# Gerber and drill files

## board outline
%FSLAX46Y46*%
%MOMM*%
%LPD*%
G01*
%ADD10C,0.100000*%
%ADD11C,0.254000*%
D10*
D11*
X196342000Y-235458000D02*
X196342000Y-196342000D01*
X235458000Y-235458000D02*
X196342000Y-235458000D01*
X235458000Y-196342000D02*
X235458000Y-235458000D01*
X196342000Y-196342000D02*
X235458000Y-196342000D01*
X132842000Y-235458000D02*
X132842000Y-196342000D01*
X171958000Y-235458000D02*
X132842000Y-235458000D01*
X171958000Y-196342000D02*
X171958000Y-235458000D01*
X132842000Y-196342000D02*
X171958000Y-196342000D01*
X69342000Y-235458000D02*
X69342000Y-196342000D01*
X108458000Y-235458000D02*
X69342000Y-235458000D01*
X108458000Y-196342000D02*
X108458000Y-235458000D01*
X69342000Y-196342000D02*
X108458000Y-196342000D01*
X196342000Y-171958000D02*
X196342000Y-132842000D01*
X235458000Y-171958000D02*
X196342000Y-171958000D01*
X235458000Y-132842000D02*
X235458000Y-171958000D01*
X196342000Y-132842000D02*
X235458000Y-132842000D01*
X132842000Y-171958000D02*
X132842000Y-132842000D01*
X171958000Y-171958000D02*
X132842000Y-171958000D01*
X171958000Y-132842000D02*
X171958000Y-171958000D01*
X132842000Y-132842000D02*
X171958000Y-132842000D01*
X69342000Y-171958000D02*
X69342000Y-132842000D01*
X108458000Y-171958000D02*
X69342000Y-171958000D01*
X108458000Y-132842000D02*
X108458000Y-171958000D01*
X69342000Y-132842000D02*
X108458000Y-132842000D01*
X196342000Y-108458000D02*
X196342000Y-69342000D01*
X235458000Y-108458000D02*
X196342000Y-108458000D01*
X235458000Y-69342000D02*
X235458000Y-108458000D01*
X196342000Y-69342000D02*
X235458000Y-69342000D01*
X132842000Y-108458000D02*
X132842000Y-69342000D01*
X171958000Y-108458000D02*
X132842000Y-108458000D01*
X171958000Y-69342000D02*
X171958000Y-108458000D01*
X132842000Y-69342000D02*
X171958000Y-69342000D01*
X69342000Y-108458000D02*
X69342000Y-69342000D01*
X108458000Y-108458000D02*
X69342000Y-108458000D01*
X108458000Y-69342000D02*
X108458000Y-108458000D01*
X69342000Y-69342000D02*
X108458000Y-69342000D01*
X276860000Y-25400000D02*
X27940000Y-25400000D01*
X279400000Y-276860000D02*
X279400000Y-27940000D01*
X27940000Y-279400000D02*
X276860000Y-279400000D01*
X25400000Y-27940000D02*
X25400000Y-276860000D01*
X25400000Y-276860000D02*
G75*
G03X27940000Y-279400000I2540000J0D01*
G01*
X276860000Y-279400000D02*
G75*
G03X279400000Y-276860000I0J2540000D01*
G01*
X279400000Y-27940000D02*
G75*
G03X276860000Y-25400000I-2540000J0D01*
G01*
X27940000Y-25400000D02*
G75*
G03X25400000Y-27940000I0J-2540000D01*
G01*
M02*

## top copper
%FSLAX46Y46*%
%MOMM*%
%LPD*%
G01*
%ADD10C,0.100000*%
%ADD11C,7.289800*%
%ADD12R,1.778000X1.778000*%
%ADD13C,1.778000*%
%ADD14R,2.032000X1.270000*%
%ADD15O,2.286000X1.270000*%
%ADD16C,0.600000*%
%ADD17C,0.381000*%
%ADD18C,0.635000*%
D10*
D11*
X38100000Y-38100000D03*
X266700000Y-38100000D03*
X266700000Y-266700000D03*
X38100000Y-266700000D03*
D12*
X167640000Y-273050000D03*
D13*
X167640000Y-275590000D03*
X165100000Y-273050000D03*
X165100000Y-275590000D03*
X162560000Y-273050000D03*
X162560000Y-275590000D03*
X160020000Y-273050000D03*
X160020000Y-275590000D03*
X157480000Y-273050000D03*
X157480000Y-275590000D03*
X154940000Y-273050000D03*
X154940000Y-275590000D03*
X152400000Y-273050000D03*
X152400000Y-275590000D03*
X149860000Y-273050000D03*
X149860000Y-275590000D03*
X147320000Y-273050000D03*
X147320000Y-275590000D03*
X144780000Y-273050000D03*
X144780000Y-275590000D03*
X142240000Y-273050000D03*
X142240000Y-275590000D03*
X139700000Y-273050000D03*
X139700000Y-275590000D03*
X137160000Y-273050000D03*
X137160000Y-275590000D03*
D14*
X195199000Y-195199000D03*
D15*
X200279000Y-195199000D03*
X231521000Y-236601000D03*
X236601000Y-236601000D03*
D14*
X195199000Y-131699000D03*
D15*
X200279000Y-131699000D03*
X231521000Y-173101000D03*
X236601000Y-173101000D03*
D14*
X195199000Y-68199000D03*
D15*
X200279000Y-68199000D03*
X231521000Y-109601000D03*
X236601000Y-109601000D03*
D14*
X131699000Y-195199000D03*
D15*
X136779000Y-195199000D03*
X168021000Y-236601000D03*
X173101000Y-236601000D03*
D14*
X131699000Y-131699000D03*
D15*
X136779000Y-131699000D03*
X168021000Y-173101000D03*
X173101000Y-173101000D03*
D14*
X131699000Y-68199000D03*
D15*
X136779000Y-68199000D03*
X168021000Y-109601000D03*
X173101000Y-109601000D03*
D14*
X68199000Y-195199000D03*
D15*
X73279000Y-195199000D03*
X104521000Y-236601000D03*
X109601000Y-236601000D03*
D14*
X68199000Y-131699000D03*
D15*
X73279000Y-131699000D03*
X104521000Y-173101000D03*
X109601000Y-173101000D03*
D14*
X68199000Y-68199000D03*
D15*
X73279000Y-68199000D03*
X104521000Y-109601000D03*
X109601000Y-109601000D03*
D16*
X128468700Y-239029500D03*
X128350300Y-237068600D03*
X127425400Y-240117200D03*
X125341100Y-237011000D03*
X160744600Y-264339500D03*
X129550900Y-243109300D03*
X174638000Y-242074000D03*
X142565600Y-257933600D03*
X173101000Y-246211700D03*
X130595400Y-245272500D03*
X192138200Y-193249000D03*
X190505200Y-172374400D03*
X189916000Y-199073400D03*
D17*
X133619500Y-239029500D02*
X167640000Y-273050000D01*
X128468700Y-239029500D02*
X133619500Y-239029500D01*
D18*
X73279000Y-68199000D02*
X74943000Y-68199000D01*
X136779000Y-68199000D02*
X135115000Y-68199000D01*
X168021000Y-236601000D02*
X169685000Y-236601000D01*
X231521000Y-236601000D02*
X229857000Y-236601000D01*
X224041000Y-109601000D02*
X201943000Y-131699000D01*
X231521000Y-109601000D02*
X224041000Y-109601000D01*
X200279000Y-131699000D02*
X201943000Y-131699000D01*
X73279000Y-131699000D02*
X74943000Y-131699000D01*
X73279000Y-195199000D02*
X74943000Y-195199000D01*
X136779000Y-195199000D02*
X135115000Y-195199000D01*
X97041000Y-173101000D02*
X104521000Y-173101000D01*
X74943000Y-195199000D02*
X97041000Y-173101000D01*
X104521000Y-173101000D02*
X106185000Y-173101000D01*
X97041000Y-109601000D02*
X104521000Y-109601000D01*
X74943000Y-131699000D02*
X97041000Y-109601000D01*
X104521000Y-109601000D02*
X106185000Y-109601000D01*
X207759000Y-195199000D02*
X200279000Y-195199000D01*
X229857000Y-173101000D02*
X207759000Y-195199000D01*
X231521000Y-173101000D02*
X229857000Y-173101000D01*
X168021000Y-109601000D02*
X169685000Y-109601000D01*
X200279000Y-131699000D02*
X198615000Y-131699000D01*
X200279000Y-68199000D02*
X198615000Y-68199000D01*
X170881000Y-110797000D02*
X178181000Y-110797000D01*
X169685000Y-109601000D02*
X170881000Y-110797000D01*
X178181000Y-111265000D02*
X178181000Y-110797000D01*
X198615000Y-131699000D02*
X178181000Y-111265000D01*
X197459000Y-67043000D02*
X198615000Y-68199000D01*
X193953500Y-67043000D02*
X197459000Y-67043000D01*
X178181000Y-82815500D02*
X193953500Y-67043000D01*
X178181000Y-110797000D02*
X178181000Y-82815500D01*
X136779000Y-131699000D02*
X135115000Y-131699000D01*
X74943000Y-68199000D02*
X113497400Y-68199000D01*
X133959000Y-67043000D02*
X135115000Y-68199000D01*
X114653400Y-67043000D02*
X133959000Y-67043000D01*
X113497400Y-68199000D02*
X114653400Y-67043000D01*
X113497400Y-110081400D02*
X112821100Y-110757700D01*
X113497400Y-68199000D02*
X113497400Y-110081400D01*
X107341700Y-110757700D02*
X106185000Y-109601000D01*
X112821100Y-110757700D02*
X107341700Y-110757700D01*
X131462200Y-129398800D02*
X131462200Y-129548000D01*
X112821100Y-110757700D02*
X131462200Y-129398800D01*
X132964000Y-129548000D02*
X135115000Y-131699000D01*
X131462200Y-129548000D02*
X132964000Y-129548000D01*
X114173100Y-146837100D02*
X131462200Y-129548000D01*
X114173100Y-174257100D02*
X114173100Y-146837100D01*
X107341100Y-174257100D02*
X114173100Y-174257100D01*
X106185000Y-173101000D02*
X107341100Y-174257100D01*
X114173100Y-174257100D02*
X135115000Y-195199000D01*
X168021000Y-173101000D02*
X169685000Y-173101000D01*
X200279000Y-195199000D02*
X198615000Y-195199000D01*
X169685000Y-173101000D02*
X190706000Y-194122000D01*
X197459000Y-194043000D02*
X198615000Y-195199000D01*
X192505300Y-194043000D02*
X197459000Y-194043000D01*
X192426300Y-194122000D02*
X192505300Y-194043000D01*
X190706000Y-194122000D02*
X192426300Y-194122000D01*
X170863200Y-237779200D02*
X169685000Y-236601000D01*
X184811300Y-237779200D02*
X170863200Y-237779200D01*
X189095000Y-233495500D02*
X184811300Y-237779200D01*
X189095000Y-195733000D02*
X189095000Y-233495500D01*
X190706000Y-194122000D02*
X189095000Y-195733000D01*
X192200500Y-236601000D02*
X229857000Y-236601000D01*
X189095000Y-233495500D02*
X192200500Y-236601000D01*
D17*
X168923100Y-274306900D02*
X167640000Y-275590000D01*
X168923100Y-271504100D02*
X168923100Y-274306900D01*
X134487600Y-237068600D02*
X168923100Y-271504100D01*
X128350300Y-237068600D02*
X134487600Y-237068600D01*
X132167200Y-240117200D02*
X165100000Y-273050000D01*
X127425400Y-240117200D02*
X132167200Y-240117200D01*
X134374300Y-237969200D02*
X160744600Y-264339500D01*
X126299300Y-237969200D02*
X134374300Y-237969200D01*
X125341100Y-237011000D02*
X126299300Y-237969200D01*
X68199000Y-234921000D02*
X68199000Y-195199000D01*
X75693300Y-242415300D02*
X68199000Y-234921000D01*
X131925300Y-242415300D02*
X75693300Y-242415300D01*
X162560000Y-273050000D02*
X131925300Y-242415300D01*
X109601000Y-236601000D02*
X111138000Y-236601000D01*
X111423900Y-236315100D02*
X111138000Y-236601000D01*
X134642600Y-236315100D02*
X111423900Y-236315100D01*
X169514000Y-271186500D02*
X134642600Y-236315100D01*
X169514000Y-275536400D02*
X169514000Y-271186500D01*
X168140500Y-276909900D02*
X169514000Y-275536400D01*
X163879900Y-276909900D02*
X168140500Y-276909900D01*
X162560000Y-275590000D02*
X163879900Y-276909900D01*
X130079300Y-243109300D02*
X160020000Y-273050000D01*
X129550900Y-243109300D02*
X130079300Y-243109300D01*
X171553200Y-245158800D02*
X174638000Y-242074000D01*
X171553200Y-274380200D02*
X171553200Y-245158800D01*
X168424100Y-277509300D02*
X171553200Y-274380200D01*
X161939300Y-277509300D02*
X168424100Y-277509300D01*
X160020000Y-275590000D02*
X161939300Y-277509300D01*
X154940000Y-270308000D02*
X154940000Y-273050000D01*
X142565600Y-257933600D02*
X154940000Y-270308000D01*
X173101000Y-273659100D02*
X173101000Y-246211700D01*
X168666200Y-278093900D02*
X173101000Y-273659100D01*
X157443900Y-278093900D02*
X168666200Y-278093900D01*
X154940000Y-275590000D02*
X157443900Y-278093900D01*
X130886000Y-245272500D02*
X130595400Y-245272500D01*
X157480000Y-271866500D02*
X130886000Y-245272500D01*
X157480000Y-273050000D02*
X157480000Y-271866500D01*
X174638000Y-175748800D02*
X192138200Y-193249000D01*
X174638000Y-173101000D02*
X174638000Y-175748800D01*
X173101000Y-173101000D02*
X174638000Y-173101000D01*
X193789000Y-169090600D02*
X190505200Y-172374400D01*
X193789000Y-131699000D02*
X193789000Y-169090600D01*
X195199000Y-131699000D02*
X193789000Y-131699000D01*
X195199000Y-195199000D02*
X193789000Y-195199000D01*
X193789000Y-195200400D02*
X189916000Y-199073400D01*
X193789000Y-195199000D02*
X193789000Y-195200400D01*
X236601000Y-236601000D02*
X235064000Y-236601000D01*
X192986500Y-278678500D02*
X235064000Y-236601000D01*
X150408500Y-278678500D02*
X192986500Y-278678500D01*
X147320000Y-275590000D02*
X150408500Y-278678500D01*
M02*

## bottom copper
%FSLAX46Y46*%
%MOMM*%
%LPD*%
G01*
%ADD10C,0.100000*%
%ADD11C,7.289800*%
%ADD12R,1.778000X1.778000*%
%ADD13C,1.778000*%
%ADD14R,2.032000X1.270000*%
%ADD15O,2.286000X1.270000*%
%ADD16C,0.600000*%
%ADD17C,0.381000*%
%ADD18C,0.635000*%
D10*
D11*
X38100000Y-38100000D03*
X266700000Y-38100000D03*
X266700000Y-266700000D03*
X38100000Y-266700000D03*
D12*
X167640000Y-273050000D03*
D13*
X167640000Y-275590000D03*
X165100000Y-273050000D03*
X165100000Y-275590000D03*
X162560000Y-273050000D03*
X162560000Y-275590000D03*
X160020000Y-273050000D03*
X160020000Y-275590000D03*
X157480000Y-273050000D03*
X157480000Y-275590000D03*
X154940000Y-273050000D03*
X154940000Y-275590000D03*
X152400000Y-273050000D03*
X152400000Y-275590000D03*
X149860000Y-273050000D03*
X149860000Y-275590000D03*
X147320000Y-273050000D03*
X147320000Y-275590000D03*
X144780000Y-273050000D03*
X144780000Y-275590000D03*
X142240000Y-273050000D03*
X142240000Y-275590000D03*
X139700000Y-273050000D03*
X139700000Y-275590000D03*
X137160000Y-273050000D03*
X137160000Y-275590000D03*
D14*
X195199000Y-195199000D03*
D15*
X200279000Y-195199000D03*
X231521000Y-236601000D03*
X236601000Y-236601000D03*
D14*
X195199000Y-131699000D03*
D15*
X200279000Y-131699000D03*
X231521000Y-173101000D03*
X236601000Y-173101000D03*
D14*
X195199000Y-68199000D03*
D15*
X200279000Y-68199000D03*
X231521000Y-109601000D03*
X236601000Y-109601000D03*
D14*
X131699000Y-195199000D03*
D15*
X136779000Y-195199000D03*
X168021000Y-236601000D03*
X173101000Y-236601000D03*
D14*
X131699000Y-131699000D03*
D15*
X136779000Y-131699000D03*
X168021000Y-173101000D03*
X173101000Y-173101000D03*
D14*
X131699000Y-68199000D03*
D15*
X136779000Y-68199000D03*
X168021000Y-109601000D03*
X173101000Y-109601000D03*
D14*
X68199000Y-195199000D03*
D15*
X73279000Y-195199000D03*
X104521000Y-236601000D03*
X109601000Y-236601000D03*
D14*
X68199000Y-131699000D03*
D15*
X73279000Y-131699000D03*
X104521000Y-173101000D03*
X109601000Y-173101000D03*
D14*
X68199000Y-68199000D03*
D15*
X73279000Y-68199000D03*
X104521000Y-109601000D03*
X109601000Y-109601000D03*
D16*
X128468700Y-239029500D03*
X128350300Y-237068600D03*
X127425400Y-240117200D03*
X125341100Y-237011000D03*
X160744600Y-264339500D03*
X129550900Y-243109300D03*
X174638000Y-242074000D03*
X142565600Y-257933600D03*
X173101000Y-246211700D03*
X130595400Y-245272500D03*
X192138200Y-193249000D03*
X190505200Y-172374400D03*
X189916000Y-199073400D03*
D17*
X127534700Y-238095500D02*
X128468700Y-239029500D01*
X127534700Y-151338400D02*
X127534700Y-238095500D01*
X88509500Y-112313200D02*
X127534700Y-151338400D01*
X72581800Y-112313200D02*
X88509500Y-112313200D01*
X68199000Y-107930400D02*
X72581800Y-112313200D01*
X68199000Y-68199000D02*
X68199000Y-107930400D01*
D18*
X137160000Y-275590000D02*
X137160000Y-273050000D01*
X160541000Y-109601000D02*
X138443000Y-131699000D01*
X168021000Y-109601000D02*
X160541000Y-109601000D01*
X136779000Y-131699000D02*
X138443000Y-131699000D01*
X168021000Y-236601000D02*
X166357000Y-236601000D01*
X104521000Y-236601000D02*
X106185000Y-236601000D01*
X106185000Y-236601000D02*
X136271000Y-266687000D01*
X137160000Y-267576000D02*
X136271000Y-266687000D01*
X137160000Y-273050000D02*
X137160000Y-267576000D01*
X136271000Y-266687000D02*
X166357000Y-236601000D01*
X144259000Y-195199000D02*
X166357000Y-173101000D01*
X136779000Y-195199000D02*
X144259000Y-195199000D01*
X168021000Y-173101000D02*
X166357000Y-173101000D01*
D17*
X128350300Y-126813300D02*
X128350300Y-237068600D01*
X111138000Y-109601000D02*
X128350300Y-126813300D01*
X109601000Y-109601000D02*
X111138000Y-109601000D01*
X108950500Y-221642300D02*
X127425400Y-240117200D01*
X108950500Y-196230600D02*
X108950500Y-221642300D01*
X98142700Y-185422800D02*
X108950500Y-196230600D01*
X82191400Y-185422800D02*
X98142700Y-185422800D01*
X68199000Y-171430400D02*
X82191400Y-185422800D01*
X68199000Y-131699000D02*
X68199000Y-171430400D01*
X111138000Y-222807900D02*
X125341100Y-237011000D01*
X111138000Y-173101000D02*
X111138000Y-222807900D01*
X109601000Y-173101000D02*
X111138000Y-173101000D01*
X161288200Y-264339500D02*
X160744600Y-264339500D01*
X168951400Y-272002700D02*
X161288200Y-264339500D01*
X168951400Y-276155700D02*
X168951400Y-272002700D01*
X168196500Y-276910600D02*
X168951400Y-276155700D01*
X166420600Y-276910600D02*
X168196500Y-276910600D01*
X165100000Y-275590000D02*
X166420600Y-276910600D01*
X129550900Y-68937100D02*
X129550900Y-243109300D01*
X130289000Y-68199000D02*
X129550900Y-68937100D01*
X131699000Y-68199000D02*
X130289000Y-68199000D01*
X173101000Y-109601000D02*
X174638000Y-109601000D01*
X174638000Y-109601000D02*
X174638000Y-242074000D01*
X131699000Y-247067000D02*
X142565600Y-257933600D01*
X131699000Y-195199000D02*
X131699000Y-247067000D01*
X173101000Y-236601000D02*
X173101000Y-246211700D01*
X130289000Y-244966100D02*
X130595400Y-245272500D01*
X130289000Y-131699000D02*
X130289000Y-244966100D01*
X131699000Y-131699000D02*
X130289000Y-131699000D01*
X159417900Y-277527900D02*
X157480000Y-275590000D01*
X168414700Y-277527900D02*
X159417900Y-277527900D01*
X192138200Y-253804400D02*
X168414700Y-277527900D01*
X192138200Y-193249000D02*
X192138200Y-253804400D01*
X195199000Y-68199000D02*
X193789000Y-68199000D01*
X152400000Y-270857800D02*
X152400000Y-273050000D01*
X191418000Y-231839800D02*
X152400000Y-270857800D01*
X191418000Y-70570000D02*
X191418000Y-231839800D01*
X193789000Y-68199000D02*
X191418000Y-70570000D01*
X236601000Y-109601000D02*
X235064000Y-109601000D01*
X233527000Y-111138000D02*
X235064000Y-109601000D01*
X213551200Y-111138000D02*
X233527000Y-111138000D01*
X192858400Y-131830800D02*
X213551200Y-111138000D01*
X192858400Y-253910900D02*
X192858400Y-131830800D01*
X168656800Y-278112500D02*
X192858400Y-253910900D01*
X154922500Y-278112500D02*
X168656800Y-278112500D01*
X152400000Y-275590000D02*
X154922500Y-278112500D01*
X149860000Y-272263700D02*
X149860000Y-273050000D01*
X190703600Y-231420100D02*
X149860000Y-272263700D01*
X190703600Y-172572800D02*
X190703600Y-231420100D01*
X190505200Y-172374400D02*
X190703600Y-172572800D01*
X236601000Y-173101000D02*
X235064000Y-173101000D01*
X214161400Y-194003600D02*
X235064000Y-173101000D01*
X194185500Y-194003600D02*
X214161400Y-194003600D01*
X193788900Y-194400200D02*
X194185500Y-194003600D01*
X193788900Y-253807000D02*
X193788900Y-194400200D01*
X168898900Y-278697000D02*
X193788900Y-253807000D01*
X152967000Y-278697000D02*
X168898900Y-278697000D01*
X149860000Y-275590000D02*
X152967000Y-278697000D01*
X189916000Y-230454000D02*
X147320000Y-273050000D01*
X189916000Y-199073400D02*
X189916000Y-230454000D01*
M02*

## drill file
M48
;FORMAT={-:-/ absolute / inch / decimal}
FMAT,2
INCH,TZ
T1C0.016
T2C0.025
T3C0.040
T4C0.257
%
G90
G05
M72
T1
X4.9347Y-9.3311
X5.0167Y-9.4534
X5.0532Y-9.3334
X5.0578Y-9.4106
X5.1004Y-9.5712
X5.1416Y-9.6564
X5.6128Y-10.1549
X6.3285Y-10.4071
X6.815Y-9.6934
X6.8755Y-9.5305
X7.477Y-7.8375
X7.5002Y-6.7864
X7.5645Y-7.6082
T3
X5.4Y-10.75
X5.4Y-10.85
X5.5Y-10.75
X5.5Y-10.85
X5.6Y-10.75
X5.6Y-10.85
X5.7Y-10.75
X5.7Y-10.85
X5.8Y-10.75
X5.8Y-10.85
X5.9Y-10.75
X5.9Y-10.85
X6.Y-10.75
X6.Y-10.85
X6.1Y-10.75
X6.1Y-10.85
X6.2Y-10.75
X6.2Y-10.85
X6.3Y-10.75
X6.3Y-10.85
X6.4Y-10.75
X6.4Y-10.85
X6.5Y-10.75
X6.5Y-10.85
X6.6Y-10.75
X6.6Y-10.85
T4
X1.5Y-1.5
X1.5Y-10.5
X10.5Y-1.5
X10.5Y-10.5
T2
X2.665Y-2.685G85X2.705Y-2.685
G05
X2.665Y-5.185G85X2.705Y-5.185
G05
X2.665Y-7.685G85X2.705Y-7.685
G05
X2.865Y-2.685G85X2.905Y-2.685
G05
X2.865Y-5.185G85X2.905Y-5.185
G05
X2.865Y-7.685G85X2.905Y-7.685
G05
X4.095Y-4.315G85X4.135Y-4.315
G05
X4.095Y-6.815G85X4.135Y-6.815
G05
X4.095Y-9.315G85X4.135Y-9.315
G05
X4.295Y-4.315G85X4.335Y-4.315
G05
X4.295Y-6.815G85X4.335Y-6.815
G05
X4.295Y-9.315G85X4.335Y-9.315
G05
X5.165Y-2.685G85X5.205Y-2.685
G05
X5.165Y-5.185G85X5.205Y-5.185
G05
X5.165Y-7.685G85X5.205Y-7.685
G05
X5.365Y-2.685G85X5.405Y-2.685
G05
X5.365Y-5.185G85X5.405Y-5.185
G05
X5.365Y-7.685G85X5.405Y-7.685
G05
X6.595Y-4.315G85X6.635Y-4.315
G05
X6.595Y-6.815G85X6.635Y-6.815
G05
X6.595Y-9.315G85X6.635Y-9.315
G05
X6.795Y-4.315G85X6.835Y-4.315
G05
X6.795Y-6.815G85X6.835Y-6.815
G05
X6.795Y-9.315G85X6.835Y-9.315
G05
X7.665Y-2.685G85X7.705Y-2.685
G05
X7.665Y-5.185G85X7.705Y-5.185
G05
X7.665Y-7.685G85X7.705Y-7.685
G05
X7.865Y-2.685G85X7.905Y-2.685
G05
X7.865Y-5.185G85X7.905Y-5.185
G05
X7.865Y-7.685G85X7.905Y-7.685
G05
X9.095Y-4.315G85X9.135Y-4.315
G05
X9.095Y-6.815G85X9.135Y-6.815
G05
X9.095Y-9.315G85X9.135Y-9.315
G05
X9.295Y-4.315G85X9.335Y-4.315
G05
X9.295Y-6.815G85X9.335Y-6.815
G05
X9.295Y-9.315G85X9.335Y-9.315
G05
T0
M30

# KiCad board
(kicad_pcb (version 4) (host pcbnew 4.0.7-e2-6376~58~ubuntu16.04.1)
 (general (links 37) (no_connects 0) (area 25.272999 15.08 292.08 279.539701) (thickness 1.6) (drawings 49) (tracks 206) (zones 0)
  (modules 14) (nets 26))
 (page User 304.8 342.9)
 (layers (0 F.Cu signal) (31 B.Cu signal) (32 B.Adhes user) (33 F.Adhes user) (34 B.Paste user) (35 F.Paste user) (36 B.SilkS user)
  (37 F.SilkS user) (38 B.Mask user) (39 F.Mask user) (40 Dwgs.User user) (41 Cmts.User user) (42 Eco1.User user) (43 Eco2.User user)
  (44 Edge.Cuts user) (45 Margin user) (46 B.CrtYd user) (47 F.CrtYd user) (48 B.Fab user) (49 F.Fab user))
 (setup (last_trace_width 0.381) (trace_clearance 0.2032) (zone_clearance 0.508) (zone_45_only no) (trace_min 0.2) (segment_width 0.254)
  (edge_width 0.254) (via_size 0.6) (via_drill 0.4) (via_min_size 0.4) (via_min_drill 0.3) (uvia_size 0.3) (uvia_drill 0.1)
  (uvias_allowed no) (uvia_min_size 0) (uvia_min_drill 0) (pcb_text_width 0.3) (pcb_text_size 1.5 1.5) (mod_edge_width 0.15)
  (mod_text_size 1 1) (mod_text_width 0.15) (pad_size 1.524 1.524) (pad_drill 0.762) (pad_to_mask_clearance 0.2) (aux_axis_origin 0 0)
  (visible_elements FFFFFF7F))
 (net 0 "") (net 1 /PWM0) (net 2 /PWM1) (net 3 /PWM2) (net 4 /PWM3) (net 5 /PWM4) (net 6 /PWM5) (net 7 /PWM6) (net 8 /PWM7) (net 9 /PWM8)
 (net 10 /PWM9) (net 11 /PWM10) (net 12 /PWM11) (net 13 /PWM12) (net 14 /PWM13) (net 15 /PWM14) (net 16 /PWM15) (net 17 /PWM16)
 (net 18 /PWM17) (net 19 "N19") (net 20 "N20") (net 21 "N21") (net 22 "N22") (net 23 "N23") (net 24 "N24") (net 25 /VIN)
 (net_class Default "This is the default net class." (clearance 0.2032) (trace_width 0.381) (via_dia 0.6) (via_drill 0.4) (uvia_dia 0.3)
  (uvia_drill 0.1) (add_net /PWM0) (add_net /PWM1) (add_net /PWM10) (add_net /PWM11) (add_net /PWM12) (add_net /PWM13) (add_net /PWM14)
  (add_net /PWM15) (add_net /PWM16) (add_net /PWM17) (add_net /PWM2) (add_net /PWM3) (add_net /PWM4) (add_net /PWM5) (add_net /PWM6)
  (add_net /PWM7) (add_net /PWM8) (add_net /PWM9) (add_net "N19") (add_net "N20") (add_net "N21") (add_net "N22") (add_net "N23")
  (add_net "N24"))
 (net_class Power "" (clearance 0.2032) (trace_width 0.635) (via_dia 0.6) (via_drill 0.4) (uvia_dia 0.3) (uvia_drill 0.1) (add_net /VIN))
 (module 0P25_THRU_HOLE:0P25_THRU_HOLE (layer F.Cu) (at 38.1 38.1)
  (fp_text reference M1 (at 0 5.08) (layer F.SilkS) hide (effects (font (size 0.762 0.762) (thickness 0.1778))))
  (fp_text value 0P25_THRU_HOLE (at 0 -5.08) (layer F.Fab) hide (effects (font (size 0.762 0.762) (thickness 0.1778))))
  (pad "" thru_hole circle (at 0 0) (size 7.2898 7.2898) (drill 6.5278) (layers *.Cu *.Mask)))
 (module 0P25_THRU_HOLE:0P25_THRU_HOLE (layer F.Cu) (at 266.7 38.1)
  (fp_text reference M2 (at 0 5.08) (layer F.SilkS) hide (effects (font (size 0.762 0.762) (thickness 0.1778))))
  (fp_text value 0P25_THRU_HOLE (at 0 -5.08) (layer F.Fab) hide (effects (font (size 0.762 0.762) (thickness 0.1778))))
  (pad "" thru_hole circle (at 0 0) (size 7.2898 7.2898) (drill 6.5278) (layers *.Cu *.Mask)))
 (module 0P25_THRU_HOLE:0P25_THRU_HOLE (layer F.Cu) (at 266.7 266.7)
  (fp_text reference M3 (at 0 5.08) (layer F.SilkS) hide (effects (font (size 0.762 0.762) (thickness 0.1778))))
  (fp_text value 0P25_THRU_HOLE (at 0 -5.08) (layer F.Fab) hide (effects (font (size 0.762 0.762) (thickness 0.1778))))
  (pad "" thru_hole circle (at 0 0) (size 7.2898 7.2898) (drill 6.5278) (layers *.Cu *.Mask)))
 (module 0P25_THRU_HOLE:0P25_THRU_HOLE (layer F.Cu) (at 38.1 266.7)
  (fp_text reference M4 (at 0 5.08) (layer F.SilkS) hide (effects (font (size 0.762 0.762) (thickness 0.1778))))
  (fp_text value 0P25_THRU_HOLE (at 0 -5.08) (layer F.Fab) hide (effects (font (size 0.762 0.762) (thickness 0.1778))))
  (pad "" thru_hole circle (at 0 0) (size 7.2898 7.2898) (drill 6.5278) (layers *.Cu *.Mask)))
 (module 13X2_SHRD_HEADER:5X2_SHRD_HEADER (layer F.Cu) (at 152.4 274.32 180)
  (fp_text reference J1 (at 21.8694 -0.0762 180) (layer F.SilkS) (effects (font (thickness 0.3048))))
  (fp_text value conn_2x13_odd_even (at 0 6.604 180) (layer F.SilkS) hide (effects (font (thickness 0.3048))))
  (pad 1 thru_hole rect (at -15.24 1.27 180) (size 1.778 1.778) (drill 1.016) (layers *.Cu *.Mask F.SilkS) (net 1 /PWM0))
  (pad 2 thru_hole circle (at -15.24 -1.27 180) (size 1.778 1.778) (drill 1.016) (layers *.Cu *.Mask F.SilkS) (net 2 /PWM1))
  (pad 3 thru_hole circle (at -12.7 1.27 180) (size 1.778 1.778) (drill 1.016) (layers *.Cu *.Mask F.SilkS) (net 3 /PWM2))
  (pad 4 thru_hole circle (at -12.7 -1.27 180) (size 1.778 1.778) (drill 1.016) (layers *.Cu *.Mask F.SilkS) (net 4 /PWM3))
  (pad 5 thru_hole circle (at -10.16 1.27 180) (size 1.778 1.778) (drill 1.016) (layers *.Cu *.Mask F.SilkS) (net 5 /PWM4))
  (pad 6 thru_hole circle (at -10.16 -1.27 180) (size 1.778 1.778) (drill 1.016) (layers *.Cu *.Mask F.SilkS) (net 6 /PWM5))
  (pad 7 thru_hole circle (at -7.62 1.27 180) (size 1.778 1.778) (drill 1.016) (layers *.Cu *.Mask F.SilkS) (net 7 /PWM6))
  (pad 8 thru_hole circle (at -7.62 -1.27 180) (size 1.778 1.778) (drill 1.016) (layers *.Cu *.Mask F.SilkS) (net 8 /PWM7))
  (pad 9 thru_hole circle (at -5.08 1.27 180) (size 1.778 1.778) (drill 1.016) (layers *.Cu *.Mask F.SilkS) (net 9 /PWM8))
  (pad 10 thru_hole circle (at -5.08 -1.27 180) (size 1.778 1.778) (drill 1.016) (layers *.Cu *.Mask F.SilkS) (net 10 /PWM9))
  (pad 11 thru_hole circle (at -2.54 1.27 180) (size 1.778 1.778) (drill 1.016) (layers *.Cu *.Mask) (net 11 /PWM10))
  (pad 12 thru_hole circle (at -2.54 -1.27 180) (size 1.778 1.778) (drill 1.016) (layers *.Cu *.Mask) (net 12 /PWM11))
  (pad 13 thru_hole circle (at 0 1.27 180) (size 1.778 1.778) (drill 1.016) (layers *.Cu *.Mask) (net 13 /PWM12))
  (pad 14 thru_hole circle (at 0 -1.27 180) (size 1.778 1.778) (drill 1.016) (layers *.Cu *.Mask) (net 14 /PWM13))
  (pad 15 thru_hole circle (at 2.54 1.27 180) (size 1.778 1.778) (drill 1.016) (layers *.Cu *.Mask) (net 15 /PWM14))
  (pad 16 thru_hole circle (at 2.54 -1.27 180) (size 1.778 1.778) (drill 1.016) (layers *.Cu *.Mask) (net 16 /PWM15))
  (pad 17 thru_hole circle (at 5.08 1.27 180) (size 1.778 1.778) (drill 1.016) (layers *.Cu *.Mask) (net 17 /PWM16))
  (pad 18 thru_hole circle (at 5.08 -1.27 180) (size 1.778 1.778) (drill 1.016) (layers *.Cu *.Mask) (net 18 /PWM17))
  (pad 19 thru_hole circle (at 7.62 1.27 180) (size 1.778 1.778) (drill 1.016) (layers *.Cu *.Mask) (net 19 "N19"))
  (pad 20 thru_hole circle (at 7.62 -1.27 180) (size 1.778 1.778) (drill 1.016) (layers *.Cu *.Mask) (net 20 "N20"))
  (pad 21 thru_hole circle (at 10.16 1.27 180) (size 1.778 1.778) (drill 1.016) (layers *.Cu *.Mask) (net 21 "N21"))
  (pad 22 thru_hole circle (at 10.16 -1.27 180) (size 1.778 1.778) (drill 1.016) (layers *.Cu *.Mask) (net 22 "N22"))
  (pad 23 thru_hole circle (at 12.7 1.27 180) (size 1.778 1.778) (drill 1.016) (layers *.Cu *.Mask) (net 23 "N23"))
  (pad 24 thru_hole circle (at 12.7 -1.27 180) (size 1.778 1.778) (drill 1.016) (layers *.Cu *.Mask) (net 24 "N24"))
  (pad 25 thru_hole circle (at 15.24 1.27 180) (size 1.778 1.778) (drill 1.016) (layers *.Cu *.Mask) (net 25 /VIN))
  (pad 26 thru_hole circle (at 15.24 -1.27 180) (size 1.778 1.778) (drill 1.016) (layers *.Cu *.Mask) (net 25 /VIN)))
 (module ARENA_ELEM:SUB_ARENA (layer F.Cu) (at 215.9 215.9)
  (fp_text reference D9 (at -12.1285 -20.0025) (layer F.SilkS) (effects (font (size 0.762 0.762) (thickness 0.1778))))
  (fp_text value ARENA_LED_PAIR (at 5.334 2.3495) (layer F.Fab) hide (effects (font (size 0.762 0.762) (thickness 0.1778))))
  (pad 1 thru_hole rect (at -20.701 -20.701) (size 2.032 1.27) (drill oval 1.651 0.635) (layers *.Cu *.Mask) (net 17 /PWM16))
  (pad 2 thru_hole oval (at -15.621 -20.701) (size 2.286 1.27) (drill oval 1.651 0.635) (layers *.Cu *.Mask) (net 25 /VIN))
  (pad 4 thru_hole oval (at 15.621 20.701) (size 2.286 1.27) (drill oval 1.651 0.635) (layers *.Cu *.Mask) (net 25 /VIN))
  (pad 3 thru_hole oval (at 20.701 20.701) (size 2.286 1.27) (drill oval 1.651 0.635) (layers *.Cu *.Mask) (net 18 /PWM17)))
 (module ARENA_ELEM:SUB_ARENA (layer F.Cu) (at 215.9 152.4)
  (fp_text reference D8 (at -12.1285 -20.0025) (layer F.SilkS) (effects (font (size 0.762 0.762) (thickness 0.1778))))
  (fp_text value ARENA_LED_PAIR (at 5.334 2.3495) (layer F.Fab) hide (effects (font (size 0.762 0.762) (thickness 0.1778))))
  (pad 1 thru_hole rect (at -20.701 -20.701) (size 2.032 1.27) (drill oval 1.651 0.635) (layers *.Cu *.Mask) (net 15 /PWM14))
  (pad 2 thru_hole oval (at -15.621 -20.701) (size 2.286 1.27) (drill oval 1.651 0.635) (layers *.Cu *.Mask) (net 25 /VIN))
  (pad 4 thru_hole oval (at 15.621 20.701) (size 2.286 1.27) (drill oval 1.651 0.635) (layers *.Cu *.Mask) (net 25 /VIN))
  (pad 3 thru_hole oval (at 20.701 20.701) (size 2.286 1.27) (drill oval 1.651 0.635) (layers *.Cu *.Mask) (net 16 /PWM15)))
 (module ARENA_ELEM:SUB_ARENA (layer F.Cu) (at 215.9 88.9)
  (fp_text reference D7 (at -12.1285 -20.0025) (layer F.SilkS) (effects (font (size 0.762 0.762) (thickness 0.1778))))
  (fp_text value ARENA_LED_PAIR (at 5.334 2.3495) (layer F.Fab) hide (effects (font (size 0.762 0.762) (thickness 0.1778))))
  (pad 1 thru_hole rect (at -20.701 -20.701) (size 2.032 1.27) (drill oval 1.651 0.635) (layers *.Cu *.Mask) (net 13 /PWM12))
  (pad 2 thru_hole oval (at -15.621 -20.701) (size 2.286 1.27) (drill oval 1.651 0.635) (layers *.Cu *.Mask) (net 25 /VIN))
  (pad 4 thru_hole oval (at 15.621 20.701) (size 2.286 1.27) (drill oval 1.651 0.635) (layers *.Cu *.Mask) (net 25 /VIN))
  (pad 3 thru_hole oval (at 20.701 20.701) (size 2.286 1.27) (drill oval 1.651 0.635) (layers *.Cu *.Mask) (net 14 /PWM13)))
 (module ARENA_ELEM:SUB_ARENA (layer F.Cu) (at 152.4 215.9)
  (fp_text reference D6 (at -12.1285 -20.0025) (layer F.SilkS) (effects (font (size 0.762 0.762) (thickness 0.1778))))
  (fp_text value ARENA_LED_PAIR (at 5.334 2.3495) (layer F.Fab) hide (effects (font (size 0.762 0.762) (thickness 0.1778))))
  (pad 1 thru_hole rect (at -20.701 -20.701) (size 2.032 1.27) (drill oval 1.651 0.635) (layers *.Cu *.Mask) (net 11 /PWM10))
  (pad 2 thru_hole oval (at -15.621 -20.701) (size 2.286 1.27) (drill oval 1.651 0.635) (layers *.Cu *.Mask) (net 25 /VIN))
  (pad 4 thru_hole oval (at 15.621 20.701) (size 2.286 1.27) (drill oval 1.651 0.635) (layers *.Cu *.Mask) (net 25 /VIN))
  (pad 3 thru_hole oval (at 20.701 20.701) (size 2.286 1.27) (drill oval 1.651 0.635) (layers *.Cu *.Mask) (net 12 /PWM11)))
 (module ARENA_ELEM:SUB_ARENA (layer F.Cu) (at 152.4 152.4)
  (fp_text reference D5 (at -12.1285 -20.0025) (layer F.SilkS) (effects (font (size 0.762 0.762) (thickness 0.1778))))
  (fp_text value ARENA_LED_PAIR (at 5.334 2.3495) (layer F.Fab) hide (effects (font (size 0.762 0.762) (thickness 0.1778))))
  (pad 1 thru_hole rect (at -20.701 -20.701) (size 2.032 1.27) (drill oval 1.651 0.635) (layers *.Cu *.Mask) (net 9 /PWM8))
  (pad 2 thru_hole oval (at -15.621 -20.701) (size 2.286 1.27) (drill oval 1.651 0.635) (layers *.Cu *.Mask) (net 25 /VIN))
  (pad 4 thru_hole oval (at 15.621 20.701) (size 2.286 1.27) (drill oval 1.651 0.635) (layers *.Cu *.Mask) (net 25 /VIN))
  (pad 3 thru_hole oval (at 20.701 20.701) (size 2.286 1.27) (drill oval 1.651 0.635) (layers *.Cu *.Mask) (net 10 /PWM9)))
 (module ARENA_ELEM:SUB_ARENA (layer F.Cu) (at 152.4 88.9)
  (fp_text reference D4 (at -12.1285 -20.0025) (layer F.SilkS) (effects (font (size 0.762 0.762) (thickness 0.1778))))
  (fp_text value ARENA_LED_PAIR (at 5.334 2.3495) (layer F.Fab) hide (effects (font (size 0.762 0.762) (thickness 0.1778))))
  (pad 1 thru_hole rect (at -20.701 -20.701) (size 2.032 1.27) (drill oval 1.651 0.635) (layers *.Cu *.Mask) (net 7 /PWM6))
  (pad 2 thru_hole oval (at -15.621 -20.701) (size 2.286 1.27) (drill oval 1.651 0.635) (layers *.Cu *.Mask) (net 25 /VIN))
  (pad 4 thru_hole oval (at 15.621 20.701) (size 2.286 1.27) (drill oval 1.651 0.635) (layers *.Cu *.Mask) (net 25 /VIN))
  (pad 3 thru_hole oval (at 20.701 20.701) (size 2.286 1.27) (drill oval 1.651 0.635) (layers *.Cu *.Mask) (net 8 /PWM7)))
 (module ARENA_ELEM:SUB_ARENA (layer F.Cu) (at 88.9 215.9)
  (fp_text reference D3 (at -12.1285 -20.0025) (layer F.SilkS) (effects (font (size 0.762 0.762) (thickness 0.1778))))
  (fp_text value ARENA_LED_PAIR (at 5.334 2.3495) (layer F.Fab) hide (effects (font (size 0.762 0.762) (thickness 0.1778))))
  (pad 1 thru_hole rect (at -20.701 -20.701) (size 2.032 1.27) (drill oval 1.651 0.635) (layers *.Cu *.Mask) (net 5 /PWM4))
  (pad 2 thru_hole oval (at -15.621 -20.701) (size 2.286 1.27) (drill oval 1.651 0.635) (layers *.Cu *.Mask) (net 25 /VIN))
  (pad 4 thru_hole oval (at 15.621 20.701) (size 2.286 1.27) (drill oval 1.651 0.635) (layers *.Cu *.Mask) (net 25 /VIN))
  (pad 3 thru_hole oval (at 20.701 20.701) (size 2.286 1.27) (drill oval 1.651 0.635) (layers *.Cu *.Mask) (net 6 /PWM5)))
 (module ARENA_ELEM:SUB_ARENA (layer F.Cu) (at 88.9 152.4)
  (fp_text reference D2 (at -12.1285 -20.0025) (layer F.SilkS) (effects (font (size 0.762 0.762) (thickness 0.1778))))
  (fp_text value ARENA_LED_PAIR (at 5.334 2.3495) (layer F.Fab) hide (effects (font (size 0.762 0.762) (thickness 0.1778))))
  (pad 1 thru_hole rect (at -20.701 -20.701) (size 2.032 1.27) (drill oval 1.651 0.635) (layers *.Cu *.Mask) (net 3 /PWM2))
  (pad 2 thru_hole oval (at -15.621 -20.701) (size 2.286 1.27) (drill oval 1.651 0.635) (layers *.Cu *.Mask) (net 25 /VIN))
  (pad 4 thru_hole oval (at 15.621 20.701) (size 2.286 1.27) (drill oval 1.651 0.635) (layers *.Cu *.Mask) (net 25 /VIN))
  (pad 3 thru_hole oval (at 20.701 20.701) (size 2.286 1.27) (drill oval 1.651 0.635) (layers *.Cu *.Mask) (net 4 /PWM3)))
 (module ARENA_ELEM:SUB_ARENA (layer F.Cu) (at 88.9 88.9)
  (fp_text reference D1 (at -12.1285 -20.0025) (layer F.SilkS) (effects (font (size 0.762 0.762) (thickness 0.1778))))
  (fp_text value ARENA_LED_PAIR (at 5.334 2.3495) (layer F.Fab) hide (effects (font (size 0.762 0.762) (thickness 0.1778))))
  (pad 1 thru_hole rect (at -20.701 -20.701) (size 2.032 1.27) (drill oval 1.651 0.635) (layers *.Cu *.Mask) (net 1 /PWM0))
  (pad 2 thru_hole oval (at -15.621 -20.701) (size 2.286 1.27) (drill oval 1.651 0.635) (layers *.Cu *.Mask) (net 25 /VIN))
  (pad 4 thru_hole oval (at 15.621 20.701) (size 2.286 1.27) (drill oval 1.651 0.635) (layers *.Cu *.Mask) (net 25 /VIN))
  (pad 3 thru_hole oval (at 20.701 20.701) (size 2.286 1.27) (drill oval 1.651 0.635) (layers *.Cu *.Mask) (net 2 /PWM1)))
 (gr_line (start 196.342 235.458) (end 196.342 196.342) (angle 90) (layer Edge.Cuts) (width 0.254))
 (gr_line (start 235.458 235.458) (end 196.342 235.458) (angle 90) (layer Edge.Cuts) (width 0.254))
 (gr_line (start 235.458 196.342) (end 235.458 235.458) (angle 90) (layer Edge.Cuts) (width 0.254))
 (gr_line (start 196.342 196.342) (end 235.458 196.342) (angle 90) (layer Edge.Cuts) (width 0.254))
 (gr_line (start 132.842 235.458) (end 132.842 196.342) (angle 90) (layer Edge.Cuts) (width 0.254))
 (gr_line (start 171.958 235.458) (end 132.842 235.458) (angle 90) (layer Edge.Cuts) (width 0.254))
 (gr_line (start 171.958 196.342) (end 171.958 235.458) (angle 90) (layer Edge.Cuts) (width 0.254))
 (gr_line (start 132.842 196.342) (end 171.958 196.342) (angle 90) (layer Edge.Cuts) (width 0.254))
 (gr_line (start 69.342 235.458) (end 69.342 196.342) (angle 90) (layer Edge.Cuts) (width 0.254))
 (gr_line (start 108.458 235.458) (end 69.342 235.458) (angle 90) (layer Edge.Cuts) (width 0.254))
 (gr_line (start 108.458 196.342) (end 108.458 235.458) (angle 90) (layer Edge.Cuts) (width 0.254))
 (gr_line (start 69.342 196.342) (end 108.458 196.342) (angle 90) (layer Edge.Cuts) (width 0.254))
 (gr_line (start 196.342 171.958) (end 196.342 132.842) (angle 90) (layer Edge.Cuts) (width 0.254))
 (gr_line (start 235.458 171.958) (end 196.342 171.958) (angle 90) (layer Edge.Cuts) (width 0.254))
 (gr_line (start 235.458 132.842) (end 235.458 171.958) (angle 90) (layer Edge.Cuts) (width 0.254))
 (gr_line (start 196.342 132.842) (end 235.458 132.842) (angle 90) (layer Edge.Cuts) (width 0.254))
 (gr_line (start 132.842 171.958) (end 132.842 132.842) (angle 90) (layer Edge.Cuts) (width 0.254))
 (gr_line (start 171.958 171.958) (end 132.842 171.958) (angle 90) (layer Edge.Cuts) (width 0.254))
 (gr_line (start 171.958 132.842) (end 171.958 171.958) (angle 90) (layer Edge.Cuts) (width 0.254))
 (gr_line (start 132.842 132.842) (end 171.958 132.842) (angle 90) (layer Edge.Cuts) (width 0.254))
 (gr_line (start 69.342 171.958) (end 69.342 132.842) (angle 90) (layer Edge.Cuts) (width 0.254))
 (gr_line (start 108.458 171.958) (end 69.342 171.958) (angle 90) (layer Edge.Cuts) (width 0.254))
 (gr_line (start 108.458 132.842) (end 108.458 171.958) (angle 90) (layer Edge.Cuts) (width 0.254))
 (gr_line (start 69.342 132.842) (end 108.458 132.842) (angle 90) (layer Edge.Cuts) (width 0.254))
 (gr_line (start 196.342 108.458) (end 196.342 69.342) (angle 90) (layer Edge.Cuts) (width 0.254))
 (gr_line (start 235.458 108.458) (end 196.342 108.458) (angle 90) (layer Edge.Cuts) (width 0.254))
 (gr_line (start 235.458 69.342) (end 235.458 108.458) (angle 90) (layer Edge.Cuts) (width 0.254))
 (gr_line (start 196.342 69.342) (end 235.458 69.342) (angle 90) (layer Edge.Cuts) (width 0.254))
 (gr_line (start 132.842 108.458) (end 132.842 69.342) (angle 90) (layer Edge.Cuts) (width 0.254))
 (gr_line (start 171.958 108.458) (end 132.842 108.458) (angle 90) (layer Edge.Cuts) (width 0.254))
 (gr_line (start 171.958 69.342) (end 171.958 108.458) (angle 90) (layer Edge.Cuts) (width 0.254))
 (gr_line (start 132.842 69.342) (end 171.958 69.342) (angle 90) (layer Edge.Cuts) (width 0.254))
 (gr_line (start 69.342 108.458) (end 69.342 69.342) (angle 90) (layer Edge.Cuts) (width 0.254))
 (gr_line (start 108.458 108.458) (end 69.342 108.458) (angle 90) (layer Edge.Cuts) (width 0.254))
 (gr_line (start 108.458 69.342) (end 108.458 108.458) (angle 90) (layer Edge.Cuts) (width 0.254))
 (gr_line (start 69.342 69.342) (end 108.458 69.342) (angle 90) (layer Edge.Cuts) (width 0.254))
 (gr_line (start 276.86 25.4) (end 27.94 25.4) (angle 90) (layer Edge.Cuts) (width 0.254))
 (gr_line (start 279.4 276.86) (end 279.4 27.94) (angle 90) (layer Edge.Cuts) (width 0.254))
 (gr_line (start 27.94 279.4) (end 276.86 279.4) (angle 90) (layer Edge.Cuts) (width 0.254))
 (gr_line (start 25.4 27.94) (end 25.4 276.86) (angle 90) (layer Edge.Cuts) (width 0.254))
 (gr_arc (start 27.94 276.86) (end 27.94 279.4) (angle 90) (layer Edge.Cuts) (width 0.254))
 (gr_arc (start 276.86 276.86) (end 279.4 276.86) (angle 90) (layer Edge.Cuts) (width 0.254))
 (gr_arc (start 276.86 27.94) (end 276.86 25.4) (angle 90) (layer Edge.Cuts) (width 0.254))
 (gr_arc (start 27.94 27.94) (end 25.4 27.94) (angle 90) (layer Edge.Cuts) (width 0.254))
 (via (at 128.4687 239.0295) (size 0.6) (layers F.Cu B.Cu) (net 1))
 (segment (start 127.5347 238.0955) (end 128.4687 239.0295) (width 0.381) (layer B.Cu) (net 1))
 (segment (start 127.5347 151.3384) (end 127.5347 238.0955) (width 0.381) (layer B.Cu) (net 1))
 (segment (start 88.5095 112.3132) (end 127.5347 151.3384) (width 0.381) (layer B.Cu) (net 1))
 (segment (start 72.5818 112.3132) (end 88.5095 112.3132) (width 0.381) (layer B.Cu) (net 1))
 (segment (start 68.199 107.9304) (end 72.5818 112.3132) (width 0.381) (layer B.Cu) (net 1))
 (segment (start 68.199 68.199) (end 68.199 107.9304) (width 0.381) (layer B.Cu) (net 1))
 (segment (start 133.6195 239.0295) (end 167.64 273.05) (width 0.381) (layer F.Cu) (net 1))
 (segment (start 128.4687 239.0295) (end 133.6195 239.0295) (width 0.381) (layer F.Cu) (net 1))
 (segment (start 73.279 68.199) (end 74.943 68.199) (width 0.635) (layer F.Cu) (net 25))
 (segment (start 136.779 68.199) (end 135.115 68.199) (width 0.635) (layer F.Cu) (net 25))
 (segment (start 137.16 275.59) (end 137.16 273.05) (width 0.635) (layer B.Cu) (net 25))
 (segment (start 168.021 236.601) (end 169.685 236.601) (width 0.635) (layer F.Cu) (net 25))
 (segment (start 231.521 236.601) (end 229.857 236.601) (width 0.635) (layer F.Cu) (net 25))
 (segment (start 224.041 109.601) (end 201.943 131.699) (width 0.635) (layer F.Cu) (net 25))
 (segment (start 231.521 109.601) (end 224.041 109.601) (width 0.635) (layer F.Cu) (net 25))
 (segment (start 200.279 131.699) (end 201.943 131.699) (width 0.635) (layer F.Cu) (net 25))
 (segment (start 73.279 131.699) (end 74.943 131.699) (width 0.635) (layer F.Cu) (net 25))
 (segment (start 73.279 195.199) (end 74.943 195.199) (width 0.635) (layer F.Cu) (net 25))
 (segment (start 136.779 195.199) (end 135.115 195.199) (width 0.635) (layer F.Cu) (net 25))
 (segment (start 97.041 173.101) (end 104.521 173.101) (width 0.635) (layer F.Cu) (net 25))
 (segment (start 74.943 195.199) (end 97.041 173.101) (width 0.635) (layer F.Cu) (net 25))
 (segment (start 104.521 173.101) (end 106.185 173.101) (width 0.635) (layer F.Cu) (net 25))
 (segment (start 97.041 109.601) (end 104.521 109.601) (width 0.635) (layer F.Cu) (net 25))
 (segment (start 74.943 131.699) (end 97.041 109.601) (width 0.635) (layer F.Cu) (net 25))
 (segment (start 104.521 109.601) (end 106.185 109.601) (width 0.635) (layer F.Cu) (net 25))
 (segment (start 160.541 109.601) (end 138.443 131.699) (width 0.635) (layer B.Cu) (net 25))
 (segment (start 168.021 109.601) (end 160.541 109.601) (width 0.635) (layer B.Cu) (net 25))
 (segment (start 136.779 131.699) (end 138.443 131.699) (width 0.635) (layer B.Cu) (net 25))
 (segment (start 207.759 195.199) (end 200.279 195.199) (width 0.635) (layer F.Cu) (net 25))
 (segment (start 229.857 173.101) (end 207.759 195.199) (width 0.635) (layer F.Cu) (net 25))
 (segment (start 231.521 173.101) (end 229.857 173.101) (width 0.635) (layer F.Cu) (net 25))
 (segment (start 168.021 109.601) (end 169.685 109.601) (width 0.635) (layer F.Cu) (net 25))
 (segment (start 200.279 131.699) (end 198.615 131.699) (width 0.635) (layer F.Cu) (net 25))
 (segment (start 200.279 68.199) (end 198.615 68.199) (width 0.635) (layer F.Cu) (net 25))
 (segment (start 170.881 110.797) (end 178.181 110.797) (width 0.635) (layer F.Cu) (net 25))
 (segment (start 169.685 109.601) (end 170.881 110.797) (width 0.635) (layer F.Cu) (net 25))
 (segment (start 178.181 111.265) (end 178.181 110.797) (width 0.635) (layer F.Cu) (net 25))
 (segment (start 198.615 131.699) (end 178.181 111.265) (width 0.635) (layer F.Cu) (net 25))
 (segment (start 197.459 67.043) (end 198.615 68.199) (width 0.635) (layer F.Cu) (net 25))
 (segment (start 193.9535 67.043) (end 197.459 67.043) (width 0.635) (layer F.Cu) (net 25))
 (segment (start 178.181 82.8155) (end 193.9535 67.043) (width 0.635) (layer F.Cu) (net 25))
 (segment (start 178.181 110.797) (end 178.181 82.8155) (width 0.635) (layer F.Cu) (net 25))
 (segment (start 136.779 131.699) (end 135.115 131.699) (width 0.635) (layer F.Cu) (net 25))
 (segment (start 74.943 68.199) (end 113.4974 68.199) (width 0.635) (layer F.Cu) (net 25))
 (segment (start 133.959 67.043) (end 135.115 68.199) (width 0.635) (layer F.Cu) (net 25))
 (segment (start 114.6534 67.043) (end 133.959 67.043) (width 0.635) (layer F.Cu) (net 25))
 (segment (start 113.4974 68.199) (end 114.6534 67.043) (width 0.635) (layer F.Cu) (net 25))
 (segment (start 113.4974 110.0814) (end 112.8211 110.7577) (width 0.635) (layer F.Cu) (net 25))
 (segment (start 113.4974 68.199) (end 113.4974 110.0814) (width 0.635) (layer F.Cu) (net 25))
 (segment (start 107.3417 110.7577) (end 106.185 109.601) (width 0.635) (layer F.Cu) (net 25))
 (segment (start 112.8211 110.7577) (end 107.3417 110.7577) (width 0.635) (layer F.Cu) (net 25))
 (segment (start 131.4622 129.3988) (end 131.4622 129.548) (width 0.635) (layer F.Cu) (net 25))
 (segment (start 112.8211 110.7577) (end 131.4622 129.3988) (width 0.635) (layer F.Cu) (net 25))
 (segment (start 132.964 129.548) (end 135.115 131.699) (width 0.635) (layer F.Cu) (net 25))
 (segment (start 131.4622 129.548) (end 132.964 129.548) (width 0.635) (layer F.Cu) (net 25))
 (segment (start 114.1731 146.8371) (end 131.4622 129.548) (width 0.635) (layer F.Cu) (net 25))
 (segment (start 114.1731 174.2571) (end 114.1731 146.8371) (width 0.635) (layer F.Cu) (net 25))
 (segment (start 107.3411 174.2571) (end 114.1731 174.2571) (width 0.635) (layer F.Cu) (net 25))
 (segment (start 106.185 173.101) (end 107.3411 174.2571) (width 0.635) (layer F.Cu) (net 25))
 (segment (start 114.1731 174.2571) (end 135.115 195.199) (width 0.635) (layer F.Cu) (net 25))
 (segment (start 168.021 236.601) (end 166.357 236.601) (width 0.635) (layer B.Cu) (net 25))
 (segment (start 104.521 236.601) (end 106.185 236.601) (width 0.635) (layer B.Cu) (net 25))
 (segment (start 106.185 236.601) (end 136.271 266.687) (width 0.635) (layer B.Cu) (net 25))
 (segment (start 137.16 267.576) (end 136.271 266.687) (width 0.635) (layer B.Cu) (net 25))
 (segment (start 137.16 273.05) (end 137.16 267.576) (width 0.635) (layer B.Cu) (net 25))
 (segment (start 136.271 266.687) (end 166.357 236.601) (width 0.635) (layer B.Cu) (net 25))
 (segment (start 144.259 195.199) (end 166.357 173.101) (width 0.635) (layer B.Cu) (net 25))
 (segment (start 136.779 195.199) (end 144.259 195.199) (width 0.635) (layer B.Cu) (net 25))
 (segment (start 168.021 173.101) (end 166.357 173.101) (width 0.635) (layer B.Cu) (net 25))
 (segment (start 168.021 173.101) (end 169.685 173.101) (width 0.635) (layer F.Cu) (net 25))
 (segment (start 200.279 195.199) (end 198.615 195.199) (width 0.635) (layer F.Cu) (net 25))
 (segment (start 169.685 173.101) (end 190.706 194.122) (width 0.635) (layer F.Cu) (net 25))
 (segment (start 197.459 194.043) (end 198.615 195.199) (width 0.635) (layer F.Cu) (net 25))
 (segment (start 192.5053 194.043) (end 197.459 194.043) (width 0.635) (layer F.Cu) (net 25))
 (segment (start 192.4263 194.122) (end 192.5053 194.043) (width 0.635) (layer F.Cu) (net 25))
 (segment (start 190.706 194.122) (end 192.4263 194.122) (width 0.635) (layer F.Cu) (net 25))
 (segment (start 170.8632 237.7792) (end 169.685 236.601) (width 0.635) (layer F.Cu) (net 25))
 (segment (start 184.8113 237.7792) (end 170.8632 237.7792) (width 0.635) (layer F.Cu) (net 25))
 (segment (start 189.095 233.4955) (end 184.8113 237.7792) (width 0.635) (layer F.Cu) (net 25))
 (segment (start 189.095 195.733) (end 189.095 233.4955) (width 0.635) (layer F.Cu) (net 25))
 (segment (start 190.706 194.122) (end 189.095 195.733) (width 0.635) (layer F.Cu) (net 25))
 (segment (start 192.2005 236.601) (end 229.857 236.601) (width 0.635) (layer F.Cu) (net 25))
 (segment (start 189.095 233.4955) (end 192.2005 236.601) (width 0.635) (layer F.Cu) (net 25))
 (via (at 128.3503 237.0686) (size 0.6) (layers F.Cu B.Cu) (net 2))
 (segment (start 128.3503 126.8133) (end 128.3503 237.0686) (width 0.381) (layer B.Cu) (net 2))
 (segment (start 111.138 109.601) (end 128.3503 126.8133) (width 0.381) (layer B.Cu) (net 2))
 (segment (start 168.9231 274.3069) (end 167.64 275.59) (width 0.381) (layer F.Cu) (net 2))
 (segment (start 168.9231 271.5041) (end 168.9231 274.3069) (width 0.381) (layer F.Cu) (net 2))
 (segment (start 134.4876 237.0686) (end 168.9231 271.5041) (width 0.381) (layer F.Cu) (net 2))
 (segment (start 128.3503 237.0686) (end 134.4876 237.0686) (width 0.381) (layer F.Cu) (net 2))
 (segment (start 109.601 109.601) (end 111.138 109.601) (width 0.381) (layer B.Cu) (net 2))
 (via (at 127.4254 240.1172) (size 0.6) (layers F.Cu B.Cu) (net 3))
 (segment (start 108.9505 221.6423) (end 127.4254 240.1172) (width 0.381) (layer B.Cu) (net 3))
 (segment (start 108.9505 196.2306) (end 108.9505 221.6423) (width 0.381) (layer B.Cu) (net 3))
 (segment (start 98.1427 185.4228) (end 108.9505 196.2306) (width 0.381) (layer B.Cu) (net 3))
 (segment (start 82.1914 185.4228) (end 98.1427 185.4228) (width 0.381) (layer B.Cu) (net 3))
 (segment (start 68.199 171.4304) (end 82.1914 185.4228) (width 0.381) (layer B.Cu) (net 3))
 (segment (start 68.199 131.699) (end 68.199 171.4304) (width 0.381) (layer B.Cu) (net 3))
 (segment (start 132.1672 240.1172) (end 165.1 273.05) (width 0.381) (layer F.Cu) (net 3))
 (segment (start 127.4254 240.1172) (end 132.1672 240.1172) (width 0.381) (layer F.Cu) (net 3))
 (via (at 125.3411 237.011) (size 0.6) (layers F.Cu B.Cu) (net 4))
 (via (at 160.7446 264.3395) (size 0.6) (layers F.Cu B.Cu) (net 4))
 (segment (start 111.138 222.8079) (end 125.3411 237.011) (width 0.381) (layer B.Cu) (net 4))
 (segment (start 111.138 173.101) (end 111.138 222.8079) (width 0.381) (layer B.Cu) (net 4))
 (segment (start 109.601 173.101) (end 111.138 173.101) (width 0.381) (layer B.Cu) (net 4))
 (segment (start 161.2882 264.3395) (end 160.7446 264.3395) (width 0.381) (layer B.Cu) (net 4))
 (segment (start 168.9514 272.0027) (end 161.2882 264.3395) (width 0.381) (layer B.Cu) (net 4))
 (segment (start 168.9514 276.1557) (end 168.9514 272.0027) (width 0.381) (layer B.Cu) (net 4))
 (segment (start 168.1965 276.9106) (end 168.9514 276.1557) (width 0.381) (layer B.Cu) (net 4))
 (segment (start 166.4206 276.9106) (end 168.1965 276.9106) (width 0.381) (layer B.Cu) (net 4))
 (segment (start 165.1 275.59) (end 166.4206 276.9106) (width 0.381) (layer B.Cu) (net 4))
 (segment (start 134.3743 237.9692) (end 160.7446 264.3395) (width 0.381) (layer F.Cu) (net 4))
 (segment (start 126.2993 237.9692) (end 134.3743 237.9692) (width 0.381) (layer F.Cu) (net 4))
 (segment (start 125.3411 237.011) (end 126.2993 237.9692) (width 0.381) (layer F.Cu) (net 4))
 (segment (start 68.199 234.921) (end 68.199 195.199) (width 0.381) (layer F.Cu) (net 5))
 (segment (start 75.6933 242.4153) (end 68.199 234.921) (width 0.381) (layer F.Cu) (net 5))
 (segment (start 131.9253 242.4153) (end 75.6933 242.4153) (width 0.381) (layer F.Cu) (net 5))
 (segment (start 162.56 273.05) (end 131.9253 242.4153) (width 0.381) (layer F.Cu) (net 5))
 (segment (start 109.601 236.601) (end 111.138 236.601) (width 0.381) (layer F.Cu) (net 6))
 (segment (start 111.4239 236.3151) (end 111.138 236.601) (width 0.381) (layer F.Cu) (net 6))
 (segment (start 134.6426 236.3151) (end 111.4239 236.3151) (width 0.381) (layer F.Cu) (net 6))
 (segment (start 169.514 271.1865) (end 134.6426 236.3151) (width 0.381) (layer F.Cu) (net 6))
 (segment (start 169.514 275.5364) (end 169.514 271.1865) (width 0.381) (layer F.Cu) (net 6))
 (segment (start 168.1405 276.9099) (end 169.514 275.5364) (width 0.381) (layer F.Cu) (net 6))
 (segment (start 163.8799 276.9099) (end 168.1405 276.9099) (width 0.381) (layer F.Cu) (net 6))
 (segment (start 162.56 275.59) (end 163.8799 276.9099) (width 0.381) (layer F.Cu) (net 6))
 (via (at 129.5509 243.1093) (size 0.6) (layers F.Cu B.Cu) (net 7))
 (segment (start 129.5509 68.9371) (end 129.5509 243.1093) (width 0.381) (layer B.Cu) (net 7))
 (segment (start 130.289 68.199) (end 129.5509 68.9371) (width 0.381) (layer B.Cu) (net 7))
 (segment (start 130.0793 243.1093) (end 160.02 273.05) (width 0.381) (layer F.Cu) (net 7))
 (segment (start 129.5509 243.1093) (end 130.0793 243.1093) (width 0.381) (layer F.Cu) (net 7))
 (segment (start 131.699 68.199) (end 130.289 68.199) (width 0.381) (layer B.Cu) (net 7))
 (via (at 174.638 242.074) (size 0.6) (layers F.Cu B.Cu) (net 8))
 (segment (start 173.101 109.601) (end 174.638 109.601) (width 0.381) (layer B.Cu) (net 8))
 (segment (start 174.638 109.601) (end 174.638 242.074) (width 0.381) (layer B.Cu) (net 8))
 (segment (start 171.5532 245.1588) (end 174.638 242.074) (width 0.381) (layer F.Cu) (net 8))
 (segment (start 171.5532 274.3802) (end 171.5532 245.1588) (width 0.381) (layer F.Cu) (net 8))
 (segment (start 168.4241 277.5093) (end 171.5532 274.3802) (width 0.381) (layer F.Cu) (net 8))
 (segment (start 161.9393 277.5093) (end 168.4241 277.5093) (width 0.381) (layer F.Cu) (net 8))
 (segment (start 160.02 275.59) (end 161.9393 277.5093) (width 0.381) (layer F.Cu) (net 8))
 (via (at 142.5656 257.9336) (size 0.6) (layers F.Cu B.Cu) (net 11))
 (segment (start 131.699 247.067) (end 142.5656 257.9336) (width 0.381) (layer B.Cu) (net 11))
 (segment (start 131.699 195.199) (end 131.699 247.067) (width 0.381) (layer B.Cu) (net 11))
 (segment (start 154.94 270.308) (end 154.94 273.05) (width 0.381) (layer F.Cu) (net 11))
 (segment (start 142.5656 257.9336) (end 154.94 270.308) (width 0.381) (layer F.Cu) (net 11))
 (via (at 173.101 246.2117) (size 0.6) (layers F.Cu B.Cu) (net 12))
 (segment (start 173.101 236.601) (end 173.101 246.2117) (width 0.381) (layer B.Cu) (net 12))
 (segment (start 173.101 273.6591) (end 173.101 246.2117) (width 0.381) (layer F.Cu) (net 12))
 (segment (start 168.6662 278.0939) (end 173.101 273.6591) (width 0.381) (layer F.Cu) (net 12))
 (segment (start 157.4439 278.0939) (end 168.6662 278.0939) (width 0.381) (layer F.Cu) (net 12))
 (segment (start 154.94 275.59) (end 157.4439 278.0939) (width 0.381) (layer F.Cu) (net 12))
 (via (at 130.5954 245.2725) (size 0.6) (layers F.Cu B.Cu) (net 9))
 (segment (start 130.289 244.9661) (end 130.5954 245.2725) (width 0.381) (layer B.Cu) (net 9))
 (segment (start 130.289 131.699) (end 130.289 244.9661) (width 0.381) (layer B.Cu) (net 9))
 (segment (start 131.699 131.699) (end 130.289 131.699) (width 0.381) (layer B.Cu) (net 9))
 (segment (start 130.886 245.2725) (end 130.5954 245.2725) (width 0.381) (layer F.Cu) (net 9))
 (segment (start 157.48 271.8665) (end 130.886 245.2725) (width 0.381) (layer F.Cu) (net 9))
 (segment (start 157.48 273.05) (end 157.48 271.8665) (width 0.381) (layer F.Cu) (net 9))
 (via (at 192.1382 193.249) (size 0.6) (layers F.Cu B.Cu) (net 10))
 (segment (start 174.638 175.7488) (end 192.1382 193.249) (width 0.381) (layer F.Cu) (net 10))
 (segment (start 174.638 173.101) (end 174.638 175.7488) (width 0.381) (layer F.Cu) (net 10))
 (segment (start 159.4179 277.5279) (end 157.48 275.59) (width 0.381) (layer B.Cu) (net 10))
 (segment (start 168.4147 277.5279) (end 159.4179 277.5279) (width 0.381) (layer B.Cu) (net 10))
 (segment (start 192.1382 253.8044) (end 168.4147 277.5279) (width 0.381) (layer B.Cu) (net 10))
 (segment (start 192.1382 193.249) (end 192.1382 253.8044) (width 0.381) (layer B.Cu) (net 10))
 (segment (start 173.101 173.101) (end 174.638 173.101) (width 0.381) (layer F.Cu) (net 10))
 (segment (start 195.199 68.199) (end 193.789 68.199) (width 0.381) (layer B.Cu) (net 13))
 (segment (start 152.4 270.8578) (end 152.4 273.05) (width 0.381) (layer B.Cu) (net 13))
 (segment (start 191.418 231.8398) (end 152.4 270.8578) (width 0.381) (layer B.Cu) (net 13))
 (segment (start 191.418 70.57) (end 191.418 231.8398) (width 0.381) (layer B.Cu) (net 13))
 (segment (start 193.789 68.199) (end 191.418 70.57) (width 0.381) (layer B.Cu) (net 13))
 (segment (start 236.601 109.601) (end 235.064 109.601) (width 0.381) (layer B.Cu) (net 14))
 (segment (start 233.527 111.138) (end 235.064 109.601) (width 0.381) (layer B.Cu) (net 14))
 (segment (start 213.5512 111.138) (end 233.527 111.138) (width 0.381) (layer B.Cu) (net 14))
 (segment (start 192.8584 131.8308) (end 213.5512 111.138) (width 0.381) (layer B.Cu) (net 14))
 (segment (start 192.8584 253.9109) (end 192.8584 131.8308) (width 0.381) (layer B.Cu) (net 14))
 (segment (start 168.6568 278.1125) (end 192.8584 253.9109) (width 0.381) (layer B.Cu) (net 14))
 (segment (start 154.9225 278.1125) (end 168.6568 278.1125) (width 0.381) (layer B.Cu) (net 14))
 (segment (start 152.4 275.59) (end 154.9225 278.1125) (width 0.381) (layer B.Cu) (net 14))
 (via (at 190.5052 172.3744) (size 0.6) (layers F.Cu B.Cu) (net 15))
 (segment (start 193.789 169.0906) (end 190.5052 172.3744) (width 0.381) (layer F.Cu) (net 15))
 (segment (start 193.789 131.699) (end 193.789 169.0906) (width 0.381) (layer F.Cu) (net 15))
 (segment (start 195.199 131.699) (end 193.789 131.699) (width 0.381) (layer F.Cu) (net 15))
 (segment (start 149.86 272.2637) (end 149.86 273.05) (width 0.381) (layer B.Cu) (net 15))
 (segment (start 190.7036 231.4201) (end 149.86 272.2637) (width 0.381) (layer B.Cu) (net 15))
 (segment (start 190.7036 172.5728) (end 190.7036 231.4201) (width 0.381) (layer B.Cu) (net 15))
 (segment (start 190.5052 172.3744) (end 190.7036 172.5728) (width 0.381) (layer B.Cu) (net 15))
 (segment (start 236.601 173.101) (end 235.064 173.101) (width 0.381) (layer B.Cu) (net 16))
 (segment (start 214.1614 194.0036) (end 235.064 173.101) (width 0.381) (layer B.Cu) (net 16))
 (segment (start 194.1855 194.0036) (end 214.1614 194.0036) (width 0.381) (layer B.Cu) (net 16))
 (segment (start 193.7889 194.4002) (end 194.1855 194.0036) (width 0.381) (layer B.Cu) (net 16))
 (segment (start 193.7889 253.807) (end 193.7889 194.4002) (width 0.381) (layer B.Cu) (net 16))
 (segment (start 168.8989 278.697) (end 193.7889 253.807) (width 0.381) (layer B.Cu) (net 16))
 (segment (start 152.967 278.697) (end 168.8989 278.697) (width 0.381) (layer B.Cu) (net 16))
 (segment (start 149.86 275.59) (end 152.967 278.697) (width 0.381) (layer B.Cu) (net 16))
 (via (at 189.916 199.0734) (size 0.6) (layers F.Cu B.Cu) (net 17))
 (segment (start 195.199 195.199) (end 193.789 195.199) (width 0.381) (layer F.Cu) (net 17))
 (segment (start 193.789 195.2004) (end 189.916 199.0734) (width 0.381) (layer F.Cu) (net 17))
 (segment (start 193.789 195.199) (end 193.789 195.2004) (width 0.381) (layer F.Cu) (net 17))
 (segment (start 189.916 230.454) (end 147.32 273.05) (width 0.381) (layer B.Cu) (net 17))
 (segment (start 189.916 199.0734) (end 189.916 230.454) (width 0.381) (layer B.Cu) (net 17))
 (segment (start 236.601 236.601) (end 235.064 236.601) (width 0.381) (layer F.Cu) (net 18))
 (segment (start 192.9865 278.6785) (end 235.064 236.601) (width 0.381) (layer F.Cu) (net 18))
 (segment (start 150.4085 278.6785) (end 192.9865 278.6785) (width 0.381) (layer F.Cu) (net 18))
 (segment (start 147.32 275.59) (end 150.4085 278.6785) (width 0.381) (layer F.Cu) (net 18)))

